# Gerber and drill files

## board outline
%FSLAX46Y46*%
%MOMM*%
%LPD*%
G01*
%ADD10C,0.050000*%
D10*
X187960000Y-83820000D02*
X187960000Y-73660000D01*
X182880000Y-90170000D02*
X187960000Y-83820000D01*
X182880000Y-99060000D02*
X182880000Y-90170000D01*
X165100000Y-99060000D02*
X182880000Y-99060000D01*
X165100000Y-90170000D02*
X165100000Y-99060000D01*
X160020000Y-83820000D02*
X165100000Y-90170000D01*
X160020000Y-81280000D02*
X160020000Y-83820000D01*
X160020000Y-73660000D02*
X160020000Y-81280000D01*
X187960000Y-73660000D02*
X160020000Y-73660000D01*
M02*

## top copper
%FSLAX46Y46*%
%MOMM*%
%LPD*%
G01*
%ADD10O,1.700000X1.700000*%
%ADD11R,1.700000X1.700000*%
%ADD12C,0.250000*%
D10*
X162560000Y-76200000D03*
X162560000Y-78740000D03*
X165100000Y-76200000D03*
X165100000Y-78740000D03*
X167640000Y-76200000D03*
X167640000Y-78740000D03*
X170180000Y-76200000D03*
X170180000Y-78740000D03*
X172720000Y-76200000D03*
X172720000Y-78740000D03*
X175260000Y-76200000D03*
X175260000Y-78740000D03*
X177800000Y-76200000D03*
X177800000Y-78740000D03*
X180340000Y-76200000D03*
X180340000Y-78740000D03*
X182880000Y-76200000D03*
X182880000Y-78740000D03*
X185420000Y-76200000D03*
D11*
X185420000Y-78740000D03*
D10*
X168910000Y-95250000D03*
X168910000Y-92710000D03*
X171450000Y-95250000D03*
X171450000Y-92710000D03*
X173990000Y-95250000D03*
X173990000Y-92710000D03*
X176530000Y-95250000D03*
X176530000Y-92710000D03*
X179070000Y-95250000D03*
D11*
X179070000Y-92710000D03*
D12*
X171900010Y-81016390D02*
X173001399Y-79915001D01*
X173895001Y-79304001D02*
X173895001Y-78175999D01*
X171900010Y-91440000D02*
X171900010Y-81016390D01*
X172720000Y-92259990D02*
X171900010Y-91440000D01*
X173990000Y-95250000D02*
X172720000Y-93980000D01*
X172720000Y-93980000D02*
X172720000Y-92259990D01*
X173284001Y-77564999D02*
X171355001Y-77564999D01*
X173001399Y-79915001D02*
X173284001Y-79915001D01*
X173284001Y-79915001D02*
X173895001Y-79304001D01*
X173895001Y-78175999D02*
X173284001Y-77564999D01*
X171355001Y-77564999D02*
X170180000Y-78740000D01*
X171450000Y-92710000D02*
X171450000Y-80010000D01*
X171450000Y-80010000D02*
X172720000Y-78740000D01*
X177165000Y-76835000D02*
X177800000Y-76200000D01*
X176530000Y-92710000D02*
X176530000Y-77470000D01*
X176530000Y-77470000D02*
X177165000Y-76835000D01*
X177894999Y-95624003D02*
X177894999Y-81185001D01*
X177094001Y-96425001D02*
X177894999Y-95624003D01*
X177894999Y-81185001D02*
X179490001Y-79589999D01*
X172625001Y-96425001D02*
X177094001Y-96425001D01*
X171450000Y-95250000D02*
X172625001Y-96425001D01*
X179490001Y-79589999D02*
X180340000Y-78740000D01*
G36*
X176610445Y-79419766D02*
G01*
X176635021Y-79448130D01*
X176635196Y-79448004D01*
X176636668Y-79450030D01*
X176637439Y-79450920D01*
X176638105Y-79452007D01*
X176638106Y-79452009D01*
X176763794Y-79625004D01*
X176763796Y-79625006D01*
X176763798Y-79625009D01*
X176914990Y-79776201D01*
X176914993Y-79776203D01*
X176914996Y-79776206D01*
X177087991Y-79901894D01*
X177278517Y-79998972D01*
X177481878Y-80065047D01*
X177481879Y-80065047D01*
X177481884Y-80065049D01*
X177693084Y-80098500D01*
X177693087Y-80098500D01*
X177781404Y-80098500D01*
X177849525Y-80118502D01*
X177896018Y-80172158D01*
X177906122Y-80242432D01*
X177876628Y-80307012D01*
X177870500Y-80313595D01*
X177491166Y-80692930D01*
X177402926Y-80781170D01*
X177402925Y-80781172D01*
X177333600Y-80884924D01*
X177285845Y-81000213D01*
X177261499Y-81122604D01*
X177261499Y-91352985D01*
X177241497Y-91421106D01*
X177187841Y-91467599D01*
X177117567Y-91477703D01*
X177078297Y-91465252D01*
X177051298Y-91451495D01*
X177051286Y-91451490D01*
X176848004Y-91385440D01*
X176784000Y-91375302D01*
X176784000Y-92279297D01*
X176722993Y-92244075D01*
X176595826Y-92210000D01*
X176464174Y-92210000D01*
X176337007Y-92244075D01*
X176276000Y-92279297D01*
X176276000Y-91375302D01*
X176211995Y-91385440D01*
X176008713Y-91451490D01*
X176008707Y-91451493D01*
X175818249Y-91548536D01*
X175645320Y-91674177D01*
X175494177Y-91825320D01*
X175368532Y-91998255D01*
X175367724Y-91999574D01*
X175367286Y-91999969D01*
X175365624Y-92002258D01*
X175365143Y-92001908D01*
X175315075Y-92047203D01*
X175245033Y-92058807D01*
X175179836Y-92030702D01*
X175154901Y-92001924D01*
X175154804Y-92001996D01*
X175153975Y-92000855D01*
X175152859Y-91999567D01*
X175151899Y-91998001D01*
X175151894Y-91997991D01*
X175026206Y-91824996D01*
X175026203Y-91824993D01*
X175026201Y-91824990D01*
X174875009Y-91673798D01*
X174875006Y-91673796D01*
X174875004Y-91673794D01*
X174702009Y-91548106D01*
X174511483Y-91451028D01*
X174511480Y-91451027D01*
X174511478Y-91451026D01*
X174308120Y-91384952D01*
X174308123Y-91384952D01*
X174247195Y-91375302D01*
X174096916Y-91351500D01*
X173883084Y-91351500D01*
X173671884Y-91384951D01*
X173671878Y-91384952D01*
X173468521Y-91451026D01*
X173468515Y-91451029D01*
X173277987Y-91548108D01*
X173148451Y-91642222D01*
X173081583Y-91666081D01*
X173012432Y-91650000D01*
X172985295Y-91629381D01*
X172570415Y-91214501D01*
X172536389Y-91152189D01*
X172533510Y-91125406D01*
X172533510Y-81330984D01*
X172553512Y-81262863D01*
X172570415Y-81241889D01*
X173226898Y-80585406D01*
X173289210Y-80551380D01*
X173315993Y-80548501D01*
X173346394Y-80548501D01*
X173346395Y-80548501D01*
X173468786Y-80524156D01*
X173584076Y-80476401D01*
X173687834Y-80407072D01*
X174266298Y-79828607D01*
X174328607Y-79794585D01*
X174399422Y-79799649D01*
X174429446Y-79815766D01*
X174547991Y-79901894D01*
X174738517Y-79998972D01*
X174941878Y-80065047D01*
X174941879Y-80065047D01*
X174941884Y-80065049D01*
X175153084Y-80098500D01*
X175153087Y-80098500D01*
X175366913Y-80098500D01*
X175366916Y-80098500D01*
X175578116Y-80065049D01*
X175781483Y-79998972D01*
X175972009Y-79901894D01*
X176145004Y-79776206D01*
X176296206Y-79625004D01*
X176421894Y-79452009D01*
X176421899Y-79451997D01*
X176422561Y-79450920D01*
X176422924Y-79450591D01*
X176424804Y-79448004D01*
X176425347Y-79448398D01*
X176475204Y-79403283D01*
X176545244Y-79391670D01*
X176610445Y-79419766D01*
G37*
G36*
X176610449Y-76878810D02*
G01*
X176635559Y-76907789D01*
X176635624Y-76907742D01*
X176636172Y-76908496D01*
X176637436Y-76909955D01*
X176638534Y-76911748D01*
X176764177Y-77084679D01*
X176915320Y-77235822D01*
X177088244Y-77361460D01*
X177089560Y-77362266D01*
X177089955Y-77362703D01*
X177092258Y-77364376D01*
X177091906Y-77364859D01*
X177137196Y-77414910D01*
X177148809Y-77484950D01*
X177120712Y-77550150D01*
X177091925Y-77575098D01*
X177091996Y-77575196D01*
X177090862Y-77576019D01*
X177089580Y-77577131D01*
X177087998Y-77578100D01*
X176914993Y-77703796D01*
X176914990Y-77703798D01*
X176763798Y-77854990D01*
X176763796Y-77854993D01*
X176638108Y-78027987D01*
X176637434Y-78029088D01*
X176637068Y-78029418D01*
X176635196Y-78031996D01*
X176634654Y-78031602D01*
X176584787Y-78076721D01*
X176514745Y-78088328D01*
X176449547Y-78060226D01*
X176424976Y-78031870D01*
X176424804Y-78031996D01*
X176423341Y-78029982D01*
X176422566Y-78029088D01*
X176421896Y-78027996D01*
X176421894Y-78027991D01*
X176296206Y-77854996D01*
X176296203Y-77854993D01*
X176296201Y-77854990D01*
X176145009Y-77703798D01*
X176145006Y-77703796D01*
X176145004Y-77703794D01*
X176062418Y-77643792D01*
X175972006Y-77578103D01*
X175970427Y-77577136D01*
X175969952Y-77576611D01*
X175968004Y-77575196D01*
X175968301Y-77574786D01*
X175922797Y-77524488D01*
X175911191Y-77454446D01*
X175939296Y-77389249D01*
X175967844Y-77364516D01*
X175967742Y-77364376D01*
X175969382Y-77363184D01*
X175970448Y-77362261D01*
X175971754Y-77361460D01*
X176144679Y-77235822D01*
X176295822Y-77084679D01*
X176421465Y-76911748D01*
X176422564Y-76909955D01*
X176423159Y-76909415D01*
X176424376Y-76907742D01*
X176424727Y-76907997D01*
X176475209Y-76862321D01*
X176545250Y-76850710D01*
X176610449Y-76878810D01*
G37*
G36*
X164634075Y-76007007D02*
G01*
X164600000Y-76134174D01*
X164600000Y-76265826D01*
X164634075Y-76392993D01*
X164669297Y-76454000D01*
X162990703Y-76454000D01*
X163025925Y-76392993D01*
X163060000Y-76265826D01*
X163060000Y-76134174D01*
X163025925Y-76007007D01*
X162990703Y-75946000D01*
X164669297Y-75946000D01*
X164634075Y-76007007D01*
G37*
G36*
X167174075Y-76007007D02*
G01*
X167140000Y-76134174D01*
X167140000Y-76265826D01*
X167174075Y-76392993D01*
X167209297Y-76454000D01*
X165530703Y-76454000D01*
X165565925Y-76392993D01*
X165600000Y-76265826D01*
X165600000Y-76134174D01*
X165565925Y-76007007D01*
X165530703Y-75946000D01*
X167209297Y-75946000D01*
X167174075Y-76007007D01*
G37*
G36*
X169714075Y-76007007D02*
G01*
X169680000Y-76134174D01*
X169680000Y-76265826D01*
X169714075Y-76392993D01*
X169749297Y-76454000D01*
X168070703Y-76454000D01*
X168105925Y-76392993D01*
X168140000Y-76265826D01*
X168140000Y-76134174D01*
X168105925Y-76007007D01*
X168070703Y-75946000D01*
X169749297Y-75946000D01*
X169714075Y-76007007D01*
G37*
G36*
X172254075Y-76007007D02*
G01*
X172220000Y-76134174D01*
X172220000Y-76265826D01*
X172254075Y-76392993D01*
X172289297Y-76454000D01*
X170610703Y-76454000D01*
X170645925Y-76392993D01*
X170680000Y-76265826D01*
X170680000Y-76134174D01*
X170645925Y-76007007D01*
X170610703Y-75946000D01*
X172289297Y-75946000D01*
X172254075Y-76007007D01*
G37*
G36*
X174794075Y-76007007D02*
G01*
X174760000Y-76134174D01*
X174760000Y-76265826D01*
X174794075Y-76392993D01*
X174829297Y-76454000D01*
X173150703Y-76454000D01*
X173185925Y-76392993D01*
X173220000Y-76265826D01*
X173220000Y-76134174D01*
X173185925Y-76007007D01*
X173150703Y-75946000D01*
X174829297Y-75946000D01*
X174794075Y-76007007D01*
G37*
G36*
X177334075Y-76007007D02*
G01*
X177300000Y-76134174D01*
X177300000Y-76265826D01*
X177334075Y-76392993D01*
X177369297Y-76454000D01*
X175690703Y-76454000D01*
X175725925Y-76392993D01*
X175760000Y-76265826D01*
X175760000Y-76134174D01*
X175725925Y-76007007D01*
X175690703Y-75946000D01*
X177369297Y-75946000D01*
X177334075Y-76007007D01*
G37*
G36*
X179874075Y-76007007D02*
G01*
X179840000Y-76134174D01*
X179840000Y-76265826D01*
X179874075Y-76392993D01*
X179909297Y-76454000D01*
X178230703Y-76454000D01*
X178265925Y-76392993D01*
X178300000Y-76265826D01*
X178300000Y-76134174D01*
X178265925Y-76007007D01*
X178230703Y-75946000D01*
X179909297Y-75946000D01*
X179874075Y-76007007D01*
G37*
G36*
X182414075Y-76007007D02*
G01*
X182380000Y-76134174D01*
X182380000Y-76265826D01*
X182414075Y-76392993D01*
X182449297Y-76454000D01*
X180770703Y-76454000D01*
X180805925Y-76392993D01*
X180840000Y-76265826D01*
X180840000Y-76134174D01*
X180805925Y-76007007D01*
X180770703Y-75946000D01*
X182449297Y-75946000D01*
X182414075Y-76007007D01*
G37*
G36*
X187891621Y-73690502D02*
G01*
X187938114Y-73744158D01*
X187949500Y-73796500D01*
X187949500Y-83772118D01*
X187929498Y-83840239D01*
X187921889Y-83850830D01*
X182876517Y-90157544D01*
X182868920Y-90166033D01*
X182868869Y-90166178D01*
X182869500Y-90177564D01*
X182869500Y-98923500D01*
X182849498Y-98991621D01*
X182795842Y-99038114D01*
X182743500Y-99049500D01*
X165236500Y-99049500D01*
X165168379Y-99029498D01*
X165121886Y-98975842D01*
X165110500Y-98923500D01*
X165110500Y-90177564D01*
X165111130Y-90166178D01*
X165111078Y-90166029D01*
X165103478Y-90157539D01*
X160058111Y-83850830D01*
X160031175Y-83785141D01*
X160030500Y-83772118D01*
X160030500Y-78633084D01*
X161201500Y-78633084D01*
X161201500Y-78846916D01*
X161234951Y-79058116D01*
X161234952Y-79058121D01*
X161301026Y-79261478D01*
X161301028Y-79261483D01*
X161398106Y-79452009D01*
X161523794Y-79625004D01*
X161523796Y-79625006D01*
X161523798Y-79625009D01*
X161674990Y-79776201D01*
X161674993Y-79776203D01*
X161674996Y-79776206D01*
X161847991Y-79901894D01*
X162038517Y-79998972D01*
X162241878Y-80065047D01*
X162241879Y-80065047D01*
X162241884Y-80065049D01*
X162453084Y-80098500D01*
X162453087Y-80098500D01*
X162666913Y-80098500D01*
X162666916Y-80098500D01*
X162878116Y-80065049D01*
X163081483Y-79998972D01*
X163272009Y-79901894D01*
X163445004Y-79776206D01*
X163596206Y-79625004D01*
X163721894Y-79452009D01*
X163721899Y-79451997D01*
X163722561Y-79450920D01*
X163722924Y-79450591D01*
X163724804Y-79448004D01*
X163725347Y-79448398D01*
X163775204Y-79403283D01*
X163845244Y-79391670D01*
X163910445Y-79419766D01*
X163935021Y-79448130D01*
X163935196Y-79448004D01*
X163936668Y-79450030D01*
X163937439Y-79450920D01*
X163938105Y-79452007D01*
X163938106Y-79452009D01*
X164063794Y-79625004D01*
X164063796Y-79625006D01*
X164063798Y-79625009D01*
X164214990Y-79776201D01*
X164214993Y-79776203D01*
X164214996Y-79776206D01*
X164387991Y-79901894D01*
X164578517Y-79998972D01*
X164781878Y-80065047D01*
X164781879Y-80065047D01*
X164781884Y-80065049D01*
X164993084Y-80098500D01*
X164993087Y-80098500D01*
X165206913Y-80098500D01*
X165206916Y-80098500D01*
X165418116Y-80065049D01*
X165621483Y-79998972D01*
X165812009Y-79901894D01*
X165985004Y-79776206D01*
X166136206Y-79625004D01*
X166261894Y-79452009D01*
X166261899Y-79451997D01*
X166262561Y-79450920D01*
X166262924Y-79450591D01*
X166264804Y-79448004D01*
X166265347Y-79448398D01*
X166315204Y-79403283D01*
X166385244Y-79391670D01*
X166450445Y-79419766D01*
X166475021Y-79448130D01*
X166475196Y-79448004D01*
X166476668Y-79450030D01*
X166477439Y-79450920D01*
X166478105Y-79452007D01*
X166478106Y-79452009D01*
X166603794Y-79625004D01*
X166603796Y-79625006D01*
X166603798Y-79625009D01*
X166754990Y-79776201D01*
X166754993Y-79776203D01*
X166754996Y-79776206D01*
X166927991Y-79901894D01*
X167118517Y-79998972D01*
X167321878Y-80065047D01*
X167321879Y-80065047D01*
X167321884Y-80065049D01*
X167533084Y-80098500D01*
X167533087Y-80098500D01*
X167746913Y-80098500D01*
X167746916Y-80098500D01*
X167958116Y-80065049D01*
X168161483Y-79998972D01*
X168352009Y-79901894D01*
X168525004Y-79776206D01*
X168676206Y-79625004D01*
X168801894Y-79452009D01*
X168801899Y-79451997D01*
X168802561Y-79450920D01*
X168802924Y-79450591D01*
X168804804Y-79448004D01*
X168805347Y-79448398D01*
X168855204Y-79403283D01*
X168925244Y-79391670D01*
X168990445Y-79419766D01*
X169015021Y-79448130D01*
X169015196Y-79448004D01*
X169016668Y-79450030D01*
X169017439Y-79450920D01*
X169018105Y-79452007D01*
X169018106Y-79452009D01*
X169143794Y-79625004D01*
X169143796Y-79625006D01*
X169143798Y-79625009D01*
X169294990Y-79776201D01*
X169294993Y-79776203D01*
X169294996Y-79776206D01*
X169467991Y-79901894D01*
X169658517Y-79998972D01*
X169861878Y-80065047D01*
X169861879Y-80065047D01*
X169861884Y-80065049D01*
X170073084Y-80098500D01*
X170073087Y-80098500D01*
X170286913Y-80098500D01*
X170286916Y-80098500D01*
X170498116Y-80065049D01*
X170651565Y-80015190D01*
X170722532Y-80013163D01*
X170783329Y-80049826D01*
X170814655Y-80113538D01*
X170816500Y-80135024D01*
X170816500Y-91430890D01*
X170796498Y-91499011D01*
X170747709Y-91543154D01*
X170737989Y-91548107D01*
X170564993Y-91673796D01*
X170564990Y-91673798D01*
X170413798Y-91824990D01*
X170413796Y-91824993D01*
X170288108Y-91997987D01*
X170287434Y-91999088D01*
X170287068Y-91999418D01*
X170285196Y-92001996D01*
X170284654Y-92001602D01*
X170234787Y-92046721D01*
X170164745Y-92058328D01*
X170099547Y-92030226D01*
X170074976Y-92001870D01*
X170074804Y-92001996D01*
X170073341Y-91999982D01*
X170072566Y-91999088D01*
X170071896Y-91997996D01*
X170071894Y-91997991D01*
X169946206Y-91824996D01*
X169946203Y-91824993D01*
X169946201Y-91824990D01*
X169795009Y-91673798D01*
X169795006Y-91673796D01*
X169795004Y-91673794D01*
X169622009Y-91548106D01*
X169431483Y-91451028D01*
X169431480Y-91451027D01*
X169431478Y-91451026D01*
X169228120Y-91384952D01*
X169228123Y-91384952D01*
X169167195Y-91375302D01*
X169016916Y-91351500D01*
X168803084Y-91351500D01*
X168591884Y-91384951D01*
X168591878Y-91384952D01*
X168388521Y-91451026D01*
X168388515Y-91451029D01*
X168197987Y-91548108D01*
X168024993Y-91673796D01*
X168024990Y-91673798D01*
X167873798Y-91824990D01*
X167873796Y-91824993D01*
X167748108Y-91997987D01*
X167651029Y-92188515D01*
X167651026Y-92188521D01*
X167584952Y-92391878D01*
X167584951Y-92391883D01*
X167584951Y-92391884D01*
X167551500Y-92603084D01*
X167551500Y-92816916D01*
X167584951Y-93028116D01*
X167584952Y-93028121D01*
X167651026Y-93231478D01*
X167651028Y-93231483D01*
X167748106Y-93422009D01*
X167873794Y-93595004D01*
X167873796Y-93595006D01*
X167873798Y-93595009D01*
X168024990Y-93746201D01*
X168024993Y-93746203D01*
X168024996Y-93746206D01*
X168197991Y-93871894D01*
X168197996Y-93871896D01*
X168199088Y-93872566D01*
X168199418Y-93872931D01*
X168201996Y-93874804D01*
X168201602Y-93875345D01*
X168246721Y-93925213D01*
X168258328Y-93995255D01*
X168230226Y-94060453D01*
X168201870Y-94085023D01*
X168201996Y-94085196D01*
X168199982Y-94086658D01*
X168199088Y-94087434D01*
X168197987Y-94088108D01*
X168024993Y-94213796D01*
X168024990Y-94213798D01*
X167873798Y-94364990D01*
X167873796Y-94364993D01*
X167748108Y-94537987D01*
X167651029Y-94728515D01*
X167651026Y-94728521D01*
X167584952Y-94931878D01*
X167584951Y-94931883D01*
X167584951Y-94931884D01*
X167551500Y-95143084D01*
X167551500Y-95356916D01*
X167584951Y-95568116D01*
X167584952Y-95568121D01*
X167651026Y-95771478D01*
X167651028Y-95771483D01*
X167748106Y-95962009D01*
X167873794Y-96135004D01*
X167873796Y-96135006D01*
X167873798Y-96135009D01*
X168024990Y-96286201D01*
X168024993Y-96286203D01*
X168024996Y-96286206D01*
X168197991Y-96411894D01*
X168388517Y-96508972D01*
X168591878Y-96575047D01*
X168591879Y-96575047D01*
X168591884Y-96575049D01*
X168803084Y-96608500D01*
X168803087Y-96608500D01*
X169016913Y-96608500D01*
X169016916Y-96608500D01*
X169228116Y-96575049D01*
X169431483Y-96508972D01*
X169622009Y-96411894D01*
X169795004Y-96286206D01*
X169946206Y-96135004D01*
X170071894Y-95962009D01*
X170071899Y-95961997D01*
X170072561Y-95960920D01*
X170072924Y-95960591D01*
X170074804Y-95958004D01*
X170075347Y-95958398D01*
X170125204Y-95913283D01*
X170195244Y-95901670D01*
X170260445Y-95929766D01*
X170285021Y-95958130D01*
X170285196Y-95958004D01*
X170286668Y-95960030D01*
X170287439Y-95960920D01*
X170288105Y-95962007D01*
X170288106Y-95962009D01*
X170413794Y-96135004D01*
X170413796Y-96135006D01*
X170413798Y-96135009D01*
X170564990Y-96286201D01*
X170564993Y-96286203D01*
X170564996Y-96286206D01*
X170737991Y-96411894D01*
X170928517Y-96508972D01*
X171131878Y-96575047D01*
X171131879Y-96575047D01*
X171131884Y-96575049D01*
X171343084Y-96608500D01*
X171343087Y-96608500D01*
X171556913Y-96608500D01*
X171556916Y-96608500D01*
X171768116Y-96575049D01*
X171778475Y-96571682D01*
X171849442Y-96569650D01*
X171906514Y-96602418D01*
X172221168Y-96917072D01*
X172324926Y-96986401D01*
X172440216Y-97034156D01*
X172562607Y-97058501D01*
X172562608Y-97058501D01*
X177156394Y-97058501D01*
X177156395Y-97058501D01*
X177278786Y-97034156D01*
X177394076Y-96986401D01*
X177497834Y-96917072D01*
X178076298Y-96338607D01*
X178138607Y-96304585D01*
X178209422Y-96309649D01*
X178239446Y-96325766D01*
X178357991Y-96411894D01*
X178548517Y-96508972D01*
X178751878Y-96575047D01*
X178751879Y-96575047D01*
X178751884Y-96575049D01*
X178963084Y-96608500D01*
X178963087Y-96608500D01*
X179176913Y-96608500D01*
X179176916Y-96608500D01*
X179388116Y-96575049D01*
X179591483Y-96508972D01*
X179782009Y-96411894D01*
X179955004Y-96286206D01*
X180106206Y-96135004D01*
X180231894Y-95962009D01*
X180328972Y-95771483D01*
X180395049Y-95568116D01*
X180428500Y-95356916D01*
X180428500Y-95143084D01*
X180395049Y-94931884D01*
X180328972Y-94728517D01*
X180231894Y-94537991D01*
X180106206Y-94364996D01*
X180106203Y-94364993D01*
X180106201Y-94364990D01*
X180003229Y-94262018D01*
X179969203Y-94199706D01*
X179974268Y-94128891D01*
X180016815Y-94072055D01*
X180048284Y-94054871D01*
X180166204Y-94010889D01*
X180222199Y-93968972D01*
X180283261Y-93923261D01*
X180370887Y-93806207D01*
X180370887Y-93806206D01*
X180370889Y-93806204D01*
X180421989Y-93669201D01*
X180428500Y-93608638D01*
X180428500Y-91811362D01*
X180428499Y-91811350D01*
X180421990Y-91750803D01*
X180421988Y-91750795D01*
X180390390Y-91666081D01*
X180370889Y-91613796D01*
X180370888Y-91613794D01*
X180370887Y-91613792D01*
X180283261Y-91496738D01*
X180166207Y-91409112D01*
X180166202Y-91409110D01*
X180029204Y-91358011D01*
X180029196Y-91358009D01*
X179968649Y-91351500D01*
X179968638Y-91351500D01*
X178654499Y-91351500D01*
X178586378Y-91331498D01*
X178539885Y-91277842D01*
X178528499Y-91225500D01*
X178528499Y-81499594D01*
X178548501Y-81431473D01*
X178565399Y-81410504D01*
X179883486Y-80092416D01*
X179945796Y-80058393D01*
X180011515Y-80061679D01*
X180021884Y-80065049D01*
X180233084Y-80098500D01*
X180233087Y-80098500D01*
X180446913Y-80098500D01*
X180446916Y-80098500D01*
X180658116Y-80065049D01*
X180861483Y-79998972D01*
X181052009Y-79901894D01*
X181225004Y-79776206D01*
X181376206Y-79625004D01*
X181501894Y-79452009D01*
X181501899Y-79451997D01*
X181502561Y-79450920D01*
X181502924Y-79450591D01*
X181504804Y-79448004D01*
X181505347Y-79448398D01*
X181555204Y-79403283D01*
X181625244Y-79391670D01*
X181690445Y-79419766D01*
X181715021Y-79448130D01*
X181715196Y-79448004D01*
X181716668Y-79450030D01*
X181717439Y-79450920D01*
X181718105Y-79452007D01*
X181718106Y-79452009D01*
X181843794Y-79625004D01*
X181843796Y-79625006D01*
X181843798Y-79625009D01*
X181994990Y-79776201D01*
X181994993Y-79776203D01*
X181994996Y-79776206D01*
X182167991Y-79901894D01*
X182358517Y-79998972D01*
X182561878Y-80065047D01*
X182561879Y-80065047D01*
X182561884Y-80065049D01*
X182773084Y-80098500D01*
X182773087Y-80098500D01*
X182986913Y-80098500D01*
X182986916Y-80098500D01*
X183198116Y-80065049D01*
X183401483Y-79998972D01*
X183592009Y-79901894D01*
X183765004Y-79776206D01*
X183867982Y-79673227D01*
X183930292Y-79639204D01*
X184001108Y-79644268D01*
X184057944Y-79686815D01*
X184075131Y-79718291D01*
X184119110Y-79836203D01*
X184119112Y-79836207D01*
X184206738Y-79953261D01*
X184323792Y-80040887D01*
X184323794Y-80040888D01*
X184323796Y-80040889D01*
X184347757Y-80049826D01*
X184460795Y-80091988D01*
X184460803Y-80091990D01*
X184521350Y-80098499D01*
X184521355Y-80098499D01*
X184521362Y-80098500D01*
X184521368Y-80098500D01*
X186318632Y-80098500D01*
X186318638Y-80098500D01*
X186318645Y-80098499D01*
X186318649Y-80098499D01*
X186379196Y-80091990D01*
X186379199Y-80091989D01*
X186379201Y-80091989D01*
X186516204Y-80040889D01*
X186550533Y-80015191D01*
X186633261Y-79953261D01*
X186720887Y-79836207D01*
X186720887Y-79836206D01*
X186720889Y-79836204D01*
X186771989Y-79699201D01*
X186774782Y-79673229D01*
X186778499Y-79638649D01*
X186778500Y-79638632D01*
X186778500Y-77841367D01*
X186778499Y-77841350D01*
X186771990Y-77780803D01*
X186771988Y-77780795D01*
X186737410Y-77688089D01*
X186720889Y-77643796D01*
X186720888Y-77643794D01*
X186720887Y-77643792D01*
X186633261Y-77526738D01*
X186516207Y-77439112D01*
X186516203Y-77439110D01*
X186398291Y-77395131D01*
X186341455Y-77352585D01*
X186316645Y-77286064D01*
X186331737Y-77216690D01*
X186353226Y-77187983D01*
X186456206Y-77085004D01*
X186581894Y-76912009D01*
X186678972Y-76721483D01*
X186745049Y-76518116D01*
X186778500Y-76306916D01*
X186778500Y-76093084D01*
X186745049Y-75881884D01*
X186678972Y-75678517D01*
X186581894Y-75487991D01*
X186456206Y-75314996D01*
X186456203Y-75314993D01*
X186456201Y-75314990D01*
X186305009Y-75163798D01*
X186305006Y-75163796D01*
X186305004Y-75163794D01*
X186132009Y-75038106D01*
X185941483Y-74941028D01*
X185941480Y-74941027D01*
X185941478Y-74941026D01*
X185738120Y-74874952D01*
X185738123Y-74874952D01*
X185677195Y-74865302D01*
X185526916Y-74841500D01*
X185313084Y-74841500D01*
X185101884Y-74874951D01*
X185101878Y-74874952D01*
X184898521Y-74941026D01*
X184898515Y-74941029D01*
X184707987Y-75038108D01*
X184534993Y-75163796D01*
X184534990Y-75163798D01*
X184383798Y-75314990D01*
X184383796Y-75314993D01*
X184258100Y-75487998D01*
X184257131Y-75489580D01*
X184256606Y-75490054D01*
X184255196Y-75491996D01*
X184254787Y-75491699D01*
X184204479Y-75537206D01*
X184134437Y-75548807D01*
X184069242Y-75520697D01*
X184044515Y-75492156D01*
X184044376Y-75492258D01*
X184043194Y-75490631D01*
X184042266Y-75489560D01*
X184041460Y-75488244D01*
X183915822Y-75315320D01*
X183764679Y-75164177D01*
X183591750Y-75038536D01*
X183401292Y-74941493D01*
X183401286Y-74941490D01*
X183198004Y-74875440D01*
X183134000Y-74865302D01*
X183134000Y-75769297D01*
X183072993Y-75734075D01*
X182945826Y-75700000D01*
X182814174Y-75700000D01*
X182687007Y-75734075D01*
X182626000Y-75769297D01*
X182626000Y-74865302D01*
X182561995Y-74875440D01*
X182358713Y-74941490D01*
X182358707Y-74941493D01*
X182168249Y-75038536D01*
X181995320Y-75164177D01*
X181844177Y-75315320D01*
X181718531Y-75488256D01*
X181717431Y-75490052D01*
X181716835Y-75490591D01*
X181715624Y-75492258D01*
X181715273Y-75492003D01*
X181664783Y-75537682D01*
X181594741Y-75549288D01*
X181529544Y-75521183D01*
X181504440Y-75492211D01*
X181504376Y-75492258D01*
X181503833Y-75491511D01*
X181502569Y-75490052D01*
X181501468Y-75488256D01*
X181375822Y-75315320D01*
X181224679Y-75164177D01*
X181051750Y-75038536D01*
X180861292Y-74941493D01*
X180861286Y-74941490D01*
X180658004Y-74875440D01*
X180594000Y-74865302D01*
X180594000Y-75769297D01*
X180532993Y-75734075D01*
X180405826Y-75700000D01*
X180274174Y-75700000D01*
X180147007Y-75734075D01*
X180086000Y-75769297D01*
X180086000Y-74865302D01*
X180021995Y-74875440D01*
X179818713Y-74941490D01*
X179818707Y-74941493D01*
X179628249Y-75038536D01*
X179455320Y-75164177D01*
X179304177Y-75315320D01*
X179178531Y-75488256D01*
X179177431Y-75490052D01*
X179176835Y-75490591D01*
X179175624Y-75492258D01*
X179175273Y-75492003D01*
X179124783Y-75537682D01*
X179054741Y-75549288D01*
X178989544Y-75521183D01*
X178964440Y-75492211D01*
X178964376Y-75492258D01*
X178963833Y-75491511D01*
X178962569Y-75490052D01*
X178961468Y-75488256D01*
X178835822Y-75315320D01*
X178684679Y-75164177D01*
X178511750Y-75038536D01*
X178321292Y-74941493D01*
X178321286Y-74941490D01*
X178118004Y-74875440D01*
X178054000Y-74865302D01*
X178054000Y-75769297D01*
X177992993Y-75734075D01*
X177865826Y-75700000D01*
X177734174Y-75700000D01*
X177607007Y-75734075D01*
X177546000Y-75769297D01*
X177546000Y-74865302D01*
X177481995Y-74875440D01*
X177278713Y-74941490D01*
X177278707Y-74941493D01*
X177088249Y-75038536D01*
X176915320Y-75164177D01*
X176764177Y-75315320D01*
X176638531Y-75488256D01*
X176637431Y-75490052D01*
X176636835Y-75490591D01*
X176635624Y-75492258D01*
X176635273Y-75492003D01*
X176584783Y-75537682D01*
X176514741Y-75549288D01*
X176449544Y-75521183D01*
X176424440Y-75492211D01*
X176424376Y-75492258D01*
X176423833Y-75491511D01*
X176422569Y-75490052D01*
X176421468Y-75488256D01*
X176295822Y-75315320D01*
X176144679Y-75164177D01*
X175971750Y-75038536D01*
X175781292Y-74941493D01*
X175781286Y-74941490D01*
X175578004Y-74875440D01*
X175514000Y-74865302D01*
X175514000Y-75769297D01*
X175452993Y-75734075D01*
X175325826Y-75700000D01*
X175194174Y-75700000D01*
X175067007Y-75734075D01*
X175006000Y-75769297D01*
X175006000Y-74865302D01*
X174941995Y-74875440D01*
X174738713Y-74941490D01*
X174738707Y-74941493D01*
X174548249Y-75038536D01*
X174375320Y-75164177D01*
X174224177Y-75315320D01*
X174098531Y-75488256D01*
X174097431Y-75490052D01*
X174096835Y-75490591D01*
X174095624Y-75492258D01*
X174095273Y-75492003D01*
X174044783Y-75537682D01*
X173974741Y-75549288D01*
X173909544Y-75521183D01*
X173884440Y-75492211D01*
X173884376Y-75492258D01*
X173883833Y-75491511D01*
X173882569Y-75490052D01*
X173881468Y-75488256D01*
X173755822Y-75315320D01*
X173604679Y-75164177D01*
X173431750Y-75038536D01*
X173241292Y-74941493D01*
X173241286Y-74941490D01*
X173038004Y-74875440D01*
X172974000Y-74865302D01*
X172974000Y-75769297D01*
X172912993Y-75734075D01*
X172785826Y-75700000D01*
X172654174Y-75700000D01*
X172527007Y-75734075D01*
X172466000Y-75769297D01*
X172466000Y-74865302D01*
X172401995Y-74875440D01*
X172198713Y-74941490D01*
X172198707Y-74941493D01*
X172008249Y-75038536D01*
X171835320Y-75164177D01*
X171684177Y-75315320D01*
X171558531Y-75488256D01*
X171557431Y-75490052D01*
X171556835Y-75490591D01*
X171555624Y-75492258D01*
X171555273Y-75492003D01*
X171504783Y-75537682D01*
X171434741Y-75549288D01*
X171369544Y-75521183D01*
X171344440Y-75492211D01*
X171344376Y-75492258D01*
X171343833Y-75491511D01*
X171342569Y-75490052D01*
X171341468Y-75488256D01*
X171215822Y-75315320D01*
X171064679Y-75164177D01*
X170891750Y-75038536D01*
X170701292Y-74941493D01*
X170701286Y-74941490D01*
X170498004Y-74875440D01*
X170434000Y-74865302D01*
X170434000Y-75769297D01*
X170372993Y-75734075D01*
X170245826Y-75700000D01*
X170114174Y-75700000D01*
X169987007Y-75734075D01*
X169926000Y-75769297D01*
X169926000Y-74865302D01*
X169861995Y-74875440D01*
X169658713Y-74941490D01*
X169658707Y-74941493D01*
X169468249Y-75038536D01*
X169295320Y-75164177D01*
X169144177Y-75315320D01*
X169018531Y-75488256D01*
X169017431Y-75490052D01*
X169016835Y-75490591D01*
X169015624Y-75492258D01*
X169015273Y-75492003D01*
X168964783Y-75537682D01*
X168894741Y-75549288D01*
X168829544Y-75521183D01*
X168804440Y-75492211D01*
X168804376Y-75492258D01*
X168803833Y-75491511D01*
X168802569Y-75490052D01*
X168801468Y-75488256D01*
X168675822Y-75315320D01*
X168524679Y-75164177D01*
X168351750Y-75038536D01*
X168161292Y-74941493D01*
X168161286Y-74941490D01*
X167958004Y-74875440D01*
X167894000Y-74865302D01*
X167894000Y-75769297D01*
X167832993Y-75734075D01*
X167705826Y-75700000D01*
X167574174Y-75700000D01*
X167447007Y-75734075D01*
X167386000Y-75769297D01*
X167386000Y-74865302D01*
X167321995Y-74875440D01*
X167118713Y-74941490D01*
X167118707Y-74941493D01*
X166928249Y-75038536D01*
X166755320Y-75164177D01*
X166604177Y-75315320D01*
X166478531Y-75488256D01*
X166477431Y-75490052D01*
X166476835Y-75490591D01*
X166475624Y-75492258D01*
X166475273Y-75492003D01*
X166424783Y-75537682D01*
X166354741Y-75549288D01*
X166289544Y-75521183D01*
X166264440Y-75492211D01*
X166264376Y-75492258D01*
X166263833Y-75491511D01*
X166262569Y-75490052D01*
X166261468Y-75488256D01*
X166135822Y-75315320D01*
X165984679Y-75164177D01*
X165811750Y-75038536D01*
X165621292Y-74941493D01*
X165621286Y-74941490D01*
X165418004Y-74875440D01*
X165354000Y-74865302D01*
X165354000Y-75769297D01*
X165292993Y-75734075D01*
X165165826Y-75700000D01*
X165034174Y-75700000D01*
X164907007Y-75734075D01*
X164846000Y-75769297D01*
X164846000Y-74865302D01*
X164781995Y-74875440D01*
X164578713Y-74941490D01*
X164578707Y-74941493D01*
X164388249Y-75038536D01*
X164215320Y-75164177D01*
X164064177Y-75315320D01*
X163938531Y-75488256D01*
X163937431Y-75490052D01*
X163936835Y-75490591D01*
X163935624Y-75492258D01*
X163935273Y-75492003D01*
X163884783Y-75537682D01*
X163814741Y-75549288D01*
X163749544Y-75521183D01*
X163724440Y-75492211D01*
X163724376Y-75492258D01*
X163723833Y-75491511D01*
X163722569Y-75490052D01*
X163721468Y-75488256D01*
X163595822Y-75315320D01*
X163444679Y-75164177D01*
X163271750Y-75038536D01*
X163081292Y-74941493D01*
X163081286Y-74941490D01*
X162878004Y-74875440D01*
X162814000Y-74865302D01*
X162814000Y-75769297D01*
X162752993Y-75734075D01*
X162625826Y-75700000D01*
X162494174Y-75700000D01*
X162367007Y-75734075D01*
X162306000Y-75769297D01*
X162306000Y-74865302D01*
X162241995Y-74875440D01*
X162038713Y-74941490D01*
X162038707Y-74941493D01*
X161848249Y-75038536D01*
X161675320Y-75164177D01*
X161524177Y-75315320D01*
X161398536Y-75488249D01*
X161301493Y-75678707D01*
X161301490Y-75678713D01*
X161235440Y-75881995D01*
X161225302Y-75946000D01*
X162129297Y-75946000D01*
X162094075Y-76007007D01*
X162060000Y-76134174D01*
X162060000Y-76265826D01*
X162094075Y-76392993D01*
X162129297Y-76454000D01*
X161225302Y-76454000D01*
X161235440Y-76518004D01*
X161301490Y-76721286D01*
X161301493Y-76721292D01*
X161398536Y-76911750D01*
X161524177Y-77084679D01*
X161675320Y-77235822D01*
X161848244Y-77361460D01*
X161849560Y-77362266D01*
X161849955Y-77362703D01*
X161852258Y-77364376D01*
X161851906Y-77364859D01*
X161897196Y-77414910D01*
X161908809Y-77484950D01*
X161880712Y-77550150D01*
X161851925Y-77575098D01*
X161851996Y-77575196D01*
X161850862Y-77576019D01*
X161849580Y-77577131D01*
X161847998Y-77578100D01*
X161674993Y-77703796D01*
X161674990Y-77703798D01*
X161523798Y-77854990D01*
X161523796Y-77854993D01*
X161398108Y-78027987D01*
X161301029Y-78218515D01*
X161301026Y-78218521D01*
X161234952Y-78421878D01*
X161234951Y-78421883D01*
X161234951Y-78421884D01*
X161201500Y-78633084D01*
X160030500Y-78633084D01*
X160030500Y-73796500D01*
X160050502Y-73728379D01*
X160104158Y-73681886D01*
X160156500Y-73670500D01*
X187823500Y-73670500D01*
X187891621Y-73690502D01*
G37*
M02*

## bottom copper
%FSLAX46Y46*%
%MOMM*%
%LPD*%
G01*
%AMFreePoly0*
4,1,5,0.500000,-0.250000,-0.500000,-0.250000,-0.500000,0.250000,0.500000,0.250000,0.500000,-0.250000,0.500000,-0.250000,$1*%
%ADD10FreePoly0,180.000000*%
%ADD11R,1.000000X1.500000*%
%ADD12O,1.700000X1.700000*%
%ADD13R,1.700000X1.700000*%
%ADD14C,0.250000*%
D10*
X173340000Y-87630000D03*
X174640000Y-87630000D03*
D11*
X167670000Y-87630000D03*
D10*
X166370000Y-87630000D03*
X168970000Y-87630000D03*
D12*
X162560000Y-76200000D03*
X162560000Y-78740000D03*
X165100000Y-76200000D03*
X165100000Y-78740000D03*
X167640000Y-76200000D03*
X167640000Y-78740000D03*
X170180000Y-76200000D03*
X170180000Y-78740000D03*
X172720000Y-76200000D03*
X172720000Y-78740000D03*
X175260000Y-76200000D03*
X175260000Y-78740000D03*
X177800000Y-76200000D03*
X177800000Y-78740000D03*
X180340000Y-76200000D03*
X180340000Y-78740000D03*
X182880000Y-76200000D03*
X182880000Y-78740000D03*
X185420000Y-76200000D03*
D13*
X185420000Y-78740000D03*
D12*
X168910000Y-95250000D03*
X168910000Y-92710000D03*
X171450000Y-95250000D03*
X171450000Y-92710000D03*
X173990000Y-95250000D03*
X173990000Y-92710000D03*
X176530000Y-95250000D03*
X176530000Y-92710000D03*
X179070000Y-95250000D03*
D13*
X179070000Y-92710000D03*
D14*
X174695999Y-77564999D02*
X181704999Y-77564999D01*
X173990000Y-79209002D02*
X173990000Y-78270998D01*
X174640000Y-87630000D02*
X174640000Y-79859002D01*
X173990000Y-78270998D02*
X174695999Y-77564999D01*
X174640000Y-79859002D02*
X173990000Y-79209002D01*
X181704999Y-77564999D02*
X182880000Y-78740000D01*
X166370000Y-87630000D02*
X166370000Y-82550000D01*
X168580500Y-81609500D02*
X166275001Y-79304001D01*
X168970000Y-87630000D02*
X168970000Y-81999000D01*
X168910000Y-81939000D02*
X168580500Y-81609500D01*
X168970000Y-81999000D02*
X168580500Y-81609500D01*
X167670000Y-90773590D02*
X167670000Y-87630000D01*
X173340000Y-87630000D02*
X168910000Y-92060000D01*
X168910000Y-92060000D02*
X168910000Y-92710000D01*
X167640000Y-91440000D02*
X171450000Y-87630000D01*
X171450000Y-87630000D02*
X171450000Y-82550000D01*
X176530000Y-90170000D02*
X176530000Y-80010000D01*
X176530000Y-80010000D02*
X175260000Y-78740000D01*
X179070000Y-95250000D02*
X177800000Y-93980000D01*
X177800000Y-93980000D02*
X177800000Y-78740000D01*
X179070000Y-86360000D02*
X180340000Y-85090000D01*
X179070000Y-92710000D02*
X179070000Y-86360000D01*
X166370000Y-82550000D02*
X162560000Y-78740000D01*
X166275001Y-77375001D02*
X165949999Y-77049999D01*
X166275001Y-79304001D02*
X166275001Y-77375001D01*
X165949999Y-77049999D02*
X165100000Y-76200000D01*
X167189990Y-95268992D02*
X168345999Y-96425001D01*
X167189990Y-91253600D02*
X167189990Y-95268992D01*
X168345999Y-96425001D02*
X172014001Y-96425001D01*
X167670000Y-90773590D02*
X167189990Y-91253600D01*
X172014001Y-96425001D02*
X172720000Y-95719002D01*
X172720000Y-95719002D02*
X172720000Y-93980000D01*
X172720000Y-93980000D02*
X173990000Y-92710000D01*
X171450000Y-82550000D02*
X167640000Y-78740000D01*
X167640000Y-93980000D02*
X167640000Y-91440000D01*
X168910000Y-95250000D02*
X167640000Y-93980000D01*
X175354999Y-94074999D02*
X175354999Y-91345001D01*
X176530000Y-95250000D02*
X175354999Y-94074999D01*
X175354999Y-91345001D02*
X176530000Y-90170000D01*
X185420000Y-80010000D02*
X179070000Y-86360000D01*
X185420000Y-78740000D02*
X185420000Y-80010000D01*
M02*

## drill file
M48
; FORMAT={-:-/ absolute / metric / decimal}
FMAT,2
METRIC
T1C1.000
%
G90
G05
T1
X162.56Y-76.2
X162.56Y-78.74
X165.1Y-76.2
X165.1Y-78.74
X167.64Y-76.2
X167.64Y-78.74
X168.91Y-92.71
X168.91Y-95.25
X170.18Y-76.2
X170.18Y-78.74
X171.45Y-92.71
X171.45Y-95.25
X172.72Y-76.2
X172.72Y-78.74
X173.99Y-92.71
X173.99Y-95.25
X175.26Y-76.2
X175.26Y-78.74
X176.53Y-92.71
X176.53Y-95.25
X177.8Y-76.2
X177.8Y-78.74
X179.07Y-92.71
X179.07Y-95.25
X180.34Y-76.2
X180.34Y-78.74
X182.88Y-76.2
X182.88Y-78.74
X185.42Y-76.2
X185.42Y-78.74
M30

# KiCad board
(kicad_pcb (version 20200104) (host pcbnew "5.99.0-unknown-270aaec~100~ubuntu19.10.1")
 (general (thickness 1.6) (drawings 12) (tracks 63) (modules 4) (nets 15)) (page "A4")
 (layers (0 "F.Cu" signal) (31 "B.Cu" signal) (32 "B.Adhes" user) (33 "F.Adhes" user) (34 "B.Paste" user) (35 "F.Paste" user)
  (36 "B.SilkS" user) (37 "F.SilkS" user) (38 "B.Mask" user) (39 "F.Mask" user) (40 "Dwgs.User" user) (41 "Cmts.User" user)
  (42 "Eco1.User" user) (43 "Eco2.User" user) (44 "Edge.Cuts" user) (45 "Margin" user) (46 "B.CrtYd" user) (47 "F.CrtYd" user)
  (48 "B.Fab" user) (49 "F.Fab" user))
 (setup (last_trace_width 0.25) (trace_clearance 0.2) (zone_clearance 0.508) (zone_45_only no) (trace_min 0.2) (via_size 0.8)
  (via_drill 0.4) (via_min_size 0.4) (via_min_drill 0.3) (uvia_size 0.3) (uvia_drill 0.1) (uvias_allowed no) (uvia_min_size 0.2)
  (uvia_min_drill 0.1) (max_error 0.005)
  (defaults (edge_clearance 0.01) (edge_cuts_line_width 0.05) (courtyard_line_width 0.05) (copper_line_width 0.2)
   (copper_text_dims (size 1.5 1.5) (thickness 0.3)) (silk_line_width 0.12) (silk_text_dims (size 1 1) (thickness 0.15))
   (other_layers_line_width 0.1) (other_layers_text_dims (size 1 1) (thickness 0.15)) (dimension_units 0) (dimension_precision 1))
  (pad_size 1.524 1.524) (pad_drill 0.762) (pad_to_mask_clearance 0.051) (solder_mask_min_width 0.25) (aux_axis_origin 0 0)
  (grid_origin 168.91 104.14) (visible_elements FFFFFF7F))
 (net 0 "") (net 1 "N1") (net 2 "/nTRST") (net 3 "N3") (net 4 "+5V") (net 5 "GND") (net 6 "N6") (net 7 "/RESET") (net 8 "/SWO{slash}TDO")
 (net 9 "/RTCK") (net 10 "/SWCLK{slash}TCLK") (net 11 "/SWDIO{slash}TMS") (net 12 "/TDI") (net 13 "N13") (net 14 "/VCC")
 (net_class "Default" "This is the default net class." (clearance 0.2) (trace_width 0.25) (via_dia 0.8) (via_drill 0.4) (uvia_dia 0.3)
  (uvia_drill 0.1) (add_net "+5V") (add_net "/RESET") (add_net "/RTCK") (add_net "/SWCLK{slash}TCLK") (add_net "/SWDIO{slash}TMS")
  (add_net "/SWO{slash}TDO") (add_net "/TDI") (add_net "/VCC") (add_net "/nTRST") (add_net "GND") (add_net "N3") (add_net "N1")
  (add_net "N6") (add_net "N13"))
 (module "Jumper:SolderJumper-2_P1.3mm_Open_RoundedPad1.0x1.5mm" (layer "B.Cu") (at 173.99 87.63 180)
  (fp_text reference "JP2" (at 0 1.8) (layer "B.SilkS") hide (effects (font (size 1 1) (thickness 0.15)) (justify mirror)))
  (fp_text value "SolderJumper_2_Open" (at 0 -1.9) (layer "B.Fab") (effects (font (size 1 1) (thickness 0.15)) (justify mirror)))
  (pad "2" smd custom (at 0.65 0 180) (size 1 0.5) (layers "B.Cu" "B.Mask") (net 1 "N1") (zone_connect 2)
   (options (clearance outline) (anchor rect)) (primitives))
  (pad "1" smd custom (at -0.65 0 180) (size 1 0.5) (layers "B.Cu" "B.Mask") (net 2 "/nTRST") (zone_connect 2)
   (options (clearance outline) (anchor rect)) (primitives)))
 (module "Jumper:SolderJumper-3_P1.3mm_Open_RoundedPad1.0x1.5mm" (layer "B.Cu") (at 167.67 87.63 180)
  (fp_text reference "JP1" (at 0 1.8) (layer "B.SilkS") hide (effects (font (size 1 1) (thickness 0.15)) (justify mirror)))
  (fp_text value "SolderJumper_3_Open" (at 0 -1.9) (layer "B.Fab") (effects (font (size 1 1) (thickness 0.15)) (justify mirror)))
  (pad "2" smd rect (at 0 0 180) (size 1 1.5) (layers "B.Cu" "B.Mask") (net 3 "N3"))
  (pad "3" smd custom (at 1.3 0 180) (size 1 0.5) (layers "B.Cu" "B.Mask") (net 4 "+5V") (zone_connect 2)
   (options (clearance outline) (anchor rect)) (primitives))
  (pad "1" smd custom (at -1.3 0 180) (size 1 0.5) (layers "B.Cu" "B.Mask") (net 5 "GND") (zone_connect 2)
   (options (clearance outline) (anchor rect)) (primitives)))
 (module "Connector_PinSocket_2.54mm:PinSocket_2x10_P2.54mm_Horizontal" (layer "F.Cu") (at 185.42 78.74 -90)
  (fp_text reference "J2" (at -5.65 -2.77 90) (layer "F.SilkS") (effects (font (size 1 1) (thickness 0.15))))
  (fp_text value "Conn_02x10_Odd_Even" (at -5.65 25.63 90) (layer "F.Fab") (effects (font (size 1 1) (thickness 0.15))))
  (pad "20" thru_hole oval (at -2.54 22.86 270) (size 1.7 1.7) (drill 1) (layers *.Cu *.Mask) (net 5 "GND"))
  (pad "19" thru_hole oval (at 0 22.86 270) (size 1.7 1.7) (drill 1) (layers *.Cu *.Mask) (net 4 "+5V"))
  (pad "18" thru_hole oval (at -2.54 20.32 270) (size 1.7 1.7) (drill 1) (layers *.Cu *.Mask) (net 5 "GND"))
  (pad "17" thru_hole oval (at 0 20.32 270) (size 1.7 1.7) (drill 1) (layers *.Cu *.Mask) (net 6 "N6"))
  (pad "16" thru_hole oval (at -2.54 17.78 270) (size 1.7 1.7) (drill 1) (layers *.Cu *.Mask) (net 5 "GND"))
  (pad "15" thru_hole oval (at 0 17.78 270) (size 1.7 1.7) (drill 1) (layers *.Cu *.Mask) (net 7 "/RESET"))
  (pad "14" thru_hole oval (at -2.54 15.24 270) (size 1.7 1.7) (drill 1) (layers *.Cu *.Mask) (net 5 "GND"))
  (pad "13" thru_hole oval (at 0 15.24 270) (size 1.7 1.7) (drill 1) (layers *.Cu *.Mask) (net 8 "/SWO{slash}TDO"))
  (pad "12" thru_hole oval (at -2.54 12.7 270) (size 1.7 1.7) (drill 1) (layers *.Cu *.Mask) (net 5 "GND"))
  (pad "11" thru_hole oval (at 0 12.7 270) (size 1.7 1.7) (drill 1) (layers *.Cu *.Mask) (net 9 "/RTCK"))
  (pad "10" thru_hole oval (at -2.54 10.16 270) (size 1.7 1.7) (drill 1) (layers *.Cu *.Mask) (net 5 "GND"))
  (pad "9" thru_hole oval (at 0 10.16 270) (size 1.7 1.7) (drill 1) (layers *.Cu *.Mask) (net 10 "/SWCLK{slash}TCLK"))
  (pad "8" thru_hole oval (at -2.54 7.62 270) (size 1.7 1.7) (drill 1) (layers *.Cu *.Mask) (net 5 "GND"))
  (pad "7" thru_hole oval (at 0 7.62 270) (size 1.7 1.7) (drill 1) (layers *.Cu *.Mask) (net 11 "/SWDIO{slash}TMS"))
  (pad "6" thru_hole oval (at -2.54 5.08 270) (size 1.7 1.7) (drill 1) (layers *.Cu *.Mask) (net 5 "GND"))
  (pad "5" thru_hole oval (at 0 5.08 270) (size 1.7 1.7) (drill 1) (layers *.Cu *.Mask) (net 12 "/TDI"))
  (pad "4" thru_hole oval (at -2.54 2.54 270) (size 1.7 1.7) (drill 1) (layers *.Cu *.Mask) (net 5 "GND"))
  (pad "3" thru_hole oval (at 0 2.54 270) (size 1.7 1.7) (drill 1) (layers *.Cu *.Mask) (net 2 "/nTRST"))
  (pad "2" thru_hole oval (at -2.54 0 270) (size 1.7 1.7) (drill 1) (layers *.Cu *.Mask) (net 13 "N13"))
  (pad "1" thru_hole rect (at 0 0 270) (size 1.7 1.7) (drill 1) (layers *.Cu *.Mask) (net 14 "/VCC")))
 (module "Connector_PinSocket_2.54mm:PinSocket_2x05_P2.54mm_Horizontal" (layer "B.Cu") (at 179.07 92.71 90)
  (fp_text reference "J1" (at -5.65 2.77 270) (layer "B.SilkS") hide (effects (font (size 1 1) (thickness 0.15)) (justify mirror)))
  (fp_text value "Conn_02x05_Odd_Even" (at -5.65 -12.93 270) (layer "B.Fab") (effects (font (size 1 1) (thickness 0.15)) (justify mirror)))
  (pad "10" thru_hole oval (at -2.54 -10.16 90) (size 1.7 1.7) (drill 1) (layers *.Cu *.Mask) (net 7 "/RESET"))
  (pad "9" thru_hole oval (at 0 -10.16 90) (size 1.7 1.7) (drill 1) (layers *.Cu *.Mask) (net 1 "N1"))
  (pad "8" thru_hole oval (at -2.54 -7.62 90) (size 1.7 1.7) (drill 1) (layers *.Cu *.Mask) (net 12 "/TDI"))
  (pad "7" thru_hole oval (at 0 -7.62 90) (size 1.7 1.7) (drill 1) (layers *.Cu *.Mask) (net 9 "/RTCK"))
  (pad "6" thru_hole oval (at -2.54 -5.08 90) (size 1.7 1.7) (drill 1) (layers *.Cu *.Mask) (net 8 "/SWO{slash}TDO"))
  (pad "5" thru_hole oval (at 0 -5.08 90) (size 1.7 1.7) (drill 1) (layers *.Cu *.Mask) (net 3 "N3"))
  (pad "4" thru_hole oval (at -2.54 -2.54 90) (size 1.7 1.7) (drill 1) (layers *.Cu *.Mask) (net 10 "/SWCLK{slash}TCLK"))
  (pad "3" thru_hole oval (at 0 -2.54 90) (size 1.7 1.7) (drill 1) (layers *.Cu *.Mask) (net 5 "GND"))
  (pad "2" thru_hole oval (at -2.54 0 90) (size 1.7 1.7) (drill 1) (layers *.Cu *.Mask) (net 11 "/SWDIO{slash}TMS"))
  (pad "1" thru_hole rect (at 0 0 90) (size 1.7 1.7) (drill 1) (layers *.Cu *.Mask) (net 14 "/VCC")))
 (gr_line (start 187.96 83.82) (end 187.96 73.66) (layer "Edge.Cuts") (width 0.05))
 (gr_line (start 182.88 90.17) (end 187.96 83.82) (layer "Edge.Cuts") (width 0.05))
 (gr_line (start 182.88 99.06) (end 182.88 90.17) (layer "Edge.Cuts") (width 0.05))
 (gr_line (start 165.1 99.06) (end 182.88 99.06) (layer "Edge.Cuts") (width 0.05))
 (gr_line (start 165.1 90.17) (end 165.1 99.06) (layer "Edge.Cuts") (width 0.05))
 (gr_line (start 160.02 83.82) (end 165.1 90.17) (layer "Edge.Cuts") (width 0.05))
 (gr_line (start 160.02 81.28) (end 160.02 83.82) (layer "Edge.Cuts") (width 0.05))
 (gr_line (start 160.02 73.66) (end 160.02 81.28) (layer "Edge.Cuts") (width 0.05))
 (gr_line (start 187.96 73.66) (end 160.02 73.66) (layer "Edge.Cuts") (width 0.05))
 (segment (start 171.90001 81.01639) (end 173.001399 79.915001) (width 0.25) (layer "F.Cu") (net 8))
 (segment (start 173.895001 79.304001) (end 173.895001 78.175999) (width 0.25) (layer "F.Cu") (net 8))
 (segment (start 171.90001 91.44) (end 171.90001 81.01639) (width 0.25) (layer "F.Cu") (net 8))
 (segment (start 172.72 92.25999) (end 171.90001 91.44) (width 0.25) (layer "F.Cu") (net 8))
 (segment (start 173.99 95.25) (end 172.72 93.98) (width 0.25) (layer "F.Cu") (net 8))
 (segment (start 172.72 93.98) (end 172.72 92.25999) (width 0.25) (layer "F.Cu") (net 8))
 (segment (start 173.284001 77.564999) (end 171.355001 77.564999) (width 0.25) (layer "F.Cu") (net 8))
 (segment (start 173.001399 79.915001) (end 173.284001 79.915001) (width 0.25) (layer "F.Cu") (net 8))
 (segment (start 173.284001 79.915001) (end 173.895001 79.304001) (width 0.25) (layer "F.Cu") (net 8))
 (segment (start 173.895001 78.175999) (end 173.284001 77.564999) (width 0.25) (layer "F.Cu") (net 8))
 (segment (start 171.355001 77.564999) (end 170.18 78.74) (width 0.25) (layer "F.Cu") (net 8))
 (segment (start 171.45 92.71) (end 171.45 80.01) (width 0.25) (layer "F.Cu") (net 9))
 (segment (start 171.45 80.01) (end 172.72 78.74) (width 0.25) (layer "F.Cu") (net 9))
 (segment (start 177.165 76.835) (end 177.8 76.2) (width 0.25) (layer "F.Cu") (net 5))
 (segment (start 176.53 92.71) (end 176.53 77.47) (width 0.25) (layer "F.Cu") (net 5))
 (segment (start 176.53 77.47) (end 177.165 76.835) (width 0.25) (layer "F.Cu") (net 5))
 (segment (start 177.894999 95.624003) (end 177.894999 81.185001) (width 0.25) (layer "F.Cu") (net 12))
 (segment (start 177.094001 96.425001) (end 177.894999 95.624003) (width 0.25) (layer "F.Cu") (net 12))
 (segment (start 177.894999 81.185001) (end 179.490001 79.589999) (width 0.25) (layer "F.Cu") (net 12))
 (segment (start 172.625001 96.425001) (end 177.094001 96.425001) (width 0.25) (layer "F.Cu") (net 12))
 (segment (start 171.45 95.25) (end 172.625001 96.425001) (width 0.25) (layer "F.Cu") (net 12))
 (segment (start 179.490001 79.589999) (end 180.34 78.74) (width 0.25) (layer "F.Cu") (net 12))
 (segment (start 174.695999 77.564999) (end 181.704999 77.564999) (width 0.25) (layer "B.Cu") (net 2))
 (segment (start 173.99 79.209002) (end 173.99 78.270998) (width 0.25) (layer "B.Cu") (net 2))
 (segment (start 174.64 87.63) (end 174.64 79.859002) (width 0.25) (layer "B.Cu") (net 2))
 (segment (start 173.99 78.270998) (end 174.695999 77.564999) (width 0.25) (layer "B.Cu") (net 2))
 (segment (start 174.64 79.859002) (end 173.99 79.209002) (width 0.25) (layer "B.Cu") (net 2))
 (segment (start 181.704999 77.564999) (end 182.88 78.74) (width 0.25) (layer "B.Cu") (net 2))
 (segment (start 166.37 87.63) (end 166.37 82.55) (width 0.25) (layer "B.Cu") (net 4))
 (segment (start 168.5805 81.6095) (end 166.275001 79.304001) (width 0.25) (layer "B.Cu") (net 5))
 (segment (start 168.97 87.63) (end 168.97 81.999) (width 0.25) (layer "B.Cu") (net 5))
 (segment (start 168.91 81.939) (end 168.5805 81.6095) (width 0.25) (layer "B.Cu") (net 5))
 (segment (start 168.97 81.999) (end 168.5805 81.6095) (width 0.25) (layer "B.Cu") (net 5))
 (segment (start 167.67 90.77359) (end 167.67 87.63) (width 0.25) (layer "B.Cu") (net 3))
 (segment (start 173.34 87.63) (end 168.91 92.06) (width 0.25) (layer "B.Cu") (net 1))
 (segment (start 168.91 92.06) (end 168.91 92.71) (width 0.25) (layer "B.Cu") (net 1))
 (segment (start 167.64 91.44) (end 171.45 87.63) (width 0.25) (layer "B.Cu") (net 7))
 (segment (start 171.45 87.63) (end 171.45 82.55) (width 0.25) (layer "B.Cu") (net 7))
 (segment (start 176.53 90.17) (end 176.53 80.01) (width 0.25) (layer "B.Cu") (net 10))
 (segment (start 176.53 80.01) (end 175.26 78.74) (width 0.25) (layer "B.Cu") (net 10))
 (segment (start 179.07 95.25) (end 177.8 93.98) (width 0.25) (layer "B.Cu") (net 11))
 (segment (start 177.8 93.98) (end 177.8 78.74) (width 0.25) (layer "B.Cu") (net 11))
 (segment (start 179.07 86.36) (end 180.34 85.09) (width 0.25) (layer "B.Cu") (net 14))
 (segment (start 179.07 92.71) (end 179.07 86.36) (width 0.25) (layer "B.Cu") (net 14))
 (segment (start 166.37 82.55) (end 162.56 78.74) (width 0.25) (layer "B.Cu") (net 4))
 (segment (start 166.275001 77.375001) (end 165.949999 77.049999) (width 0.25) (layer "B.Cu") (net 5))
 (segment (start 166.275001 79.304001) (end 166.275001 77.375001) (width 0.25) (layer "B.Cu") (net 5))
 (segment (start 165.949999 77.049999) (end 165.1 76.2) (width 0.25) (layer "B.Cu") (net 5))
 (segment (start 167.18999 95.268992) (end 168.345999 96.425001) (width 0.25) (layer "B.Cu") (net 3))
 (segment (start 167.18999 91.2536) (end 167.18999 95.268992) (width 0.25) (layer "B.Cu") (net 3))
 (segment (start 168.345999 96.425001) (end 172.014001 96.425001) (width 0.25) (layer "B.Cu") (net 3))
 (segment (start 167.67 90.77359) (end 167.18999 91.2536) (width 0.25) (layer "B.Cu") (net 3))
 (segment (start 172.014001 96.425001) (end 172.72 95.719002) (width 0.25) (layer "B.Cu") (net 3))
 (segment (start 172.72 95.719002) (end 172.72 93.98) (width 0.25) (layer "B.Cu") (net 3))
 (segment (start 172.72 93.98) (end 173.99 92.71) (width 0.25) (layer "B.Cu") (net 3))
 (segment (start 171.45 82.55) (end 167.64 78.74) (width 0.25) (layer "B.Cu") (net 7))
 (segment (start 167.64 93.98) (end 167.64 91.44) (width 0.25) (layer "B.Cu") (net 7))
 (segment (start 168.91 95.25) (end 167.64 93.98) (width 0.25) (layer "B.Cu") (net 7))
 (segment (start 175.354999 94.074999) (end 175.354999 91.345001) (width 0.25) (layer "B.Cu") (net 10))
 (segment (start 176.53 95.25) (end 175.354999 94.074999) (width 0.25) (layer "B.Cu") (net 10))
 (segment (start 175.354999 91.345001) (end 176.53 90.17) (width 0.25) (layer "B.Cu") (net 10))
 (segment (start 185.42 80.01) (end 179.07 86.36) (width 0.25) (layer "B.Cu") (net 14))
 (segment (start 185.42 78.74) (end 185.42 80.01) (width 0.25) (layer "B.Cu") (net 14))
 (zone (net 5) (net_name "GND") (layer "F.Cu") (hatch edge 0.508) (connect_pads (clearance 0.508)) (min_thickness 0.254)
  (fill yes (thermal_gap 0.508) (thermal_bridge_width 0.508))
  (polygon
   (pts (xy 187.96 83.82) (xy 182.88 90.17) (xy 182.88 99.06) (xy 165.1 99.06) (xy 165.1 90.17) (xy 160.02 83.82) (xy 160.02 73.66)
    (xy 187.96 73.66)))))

